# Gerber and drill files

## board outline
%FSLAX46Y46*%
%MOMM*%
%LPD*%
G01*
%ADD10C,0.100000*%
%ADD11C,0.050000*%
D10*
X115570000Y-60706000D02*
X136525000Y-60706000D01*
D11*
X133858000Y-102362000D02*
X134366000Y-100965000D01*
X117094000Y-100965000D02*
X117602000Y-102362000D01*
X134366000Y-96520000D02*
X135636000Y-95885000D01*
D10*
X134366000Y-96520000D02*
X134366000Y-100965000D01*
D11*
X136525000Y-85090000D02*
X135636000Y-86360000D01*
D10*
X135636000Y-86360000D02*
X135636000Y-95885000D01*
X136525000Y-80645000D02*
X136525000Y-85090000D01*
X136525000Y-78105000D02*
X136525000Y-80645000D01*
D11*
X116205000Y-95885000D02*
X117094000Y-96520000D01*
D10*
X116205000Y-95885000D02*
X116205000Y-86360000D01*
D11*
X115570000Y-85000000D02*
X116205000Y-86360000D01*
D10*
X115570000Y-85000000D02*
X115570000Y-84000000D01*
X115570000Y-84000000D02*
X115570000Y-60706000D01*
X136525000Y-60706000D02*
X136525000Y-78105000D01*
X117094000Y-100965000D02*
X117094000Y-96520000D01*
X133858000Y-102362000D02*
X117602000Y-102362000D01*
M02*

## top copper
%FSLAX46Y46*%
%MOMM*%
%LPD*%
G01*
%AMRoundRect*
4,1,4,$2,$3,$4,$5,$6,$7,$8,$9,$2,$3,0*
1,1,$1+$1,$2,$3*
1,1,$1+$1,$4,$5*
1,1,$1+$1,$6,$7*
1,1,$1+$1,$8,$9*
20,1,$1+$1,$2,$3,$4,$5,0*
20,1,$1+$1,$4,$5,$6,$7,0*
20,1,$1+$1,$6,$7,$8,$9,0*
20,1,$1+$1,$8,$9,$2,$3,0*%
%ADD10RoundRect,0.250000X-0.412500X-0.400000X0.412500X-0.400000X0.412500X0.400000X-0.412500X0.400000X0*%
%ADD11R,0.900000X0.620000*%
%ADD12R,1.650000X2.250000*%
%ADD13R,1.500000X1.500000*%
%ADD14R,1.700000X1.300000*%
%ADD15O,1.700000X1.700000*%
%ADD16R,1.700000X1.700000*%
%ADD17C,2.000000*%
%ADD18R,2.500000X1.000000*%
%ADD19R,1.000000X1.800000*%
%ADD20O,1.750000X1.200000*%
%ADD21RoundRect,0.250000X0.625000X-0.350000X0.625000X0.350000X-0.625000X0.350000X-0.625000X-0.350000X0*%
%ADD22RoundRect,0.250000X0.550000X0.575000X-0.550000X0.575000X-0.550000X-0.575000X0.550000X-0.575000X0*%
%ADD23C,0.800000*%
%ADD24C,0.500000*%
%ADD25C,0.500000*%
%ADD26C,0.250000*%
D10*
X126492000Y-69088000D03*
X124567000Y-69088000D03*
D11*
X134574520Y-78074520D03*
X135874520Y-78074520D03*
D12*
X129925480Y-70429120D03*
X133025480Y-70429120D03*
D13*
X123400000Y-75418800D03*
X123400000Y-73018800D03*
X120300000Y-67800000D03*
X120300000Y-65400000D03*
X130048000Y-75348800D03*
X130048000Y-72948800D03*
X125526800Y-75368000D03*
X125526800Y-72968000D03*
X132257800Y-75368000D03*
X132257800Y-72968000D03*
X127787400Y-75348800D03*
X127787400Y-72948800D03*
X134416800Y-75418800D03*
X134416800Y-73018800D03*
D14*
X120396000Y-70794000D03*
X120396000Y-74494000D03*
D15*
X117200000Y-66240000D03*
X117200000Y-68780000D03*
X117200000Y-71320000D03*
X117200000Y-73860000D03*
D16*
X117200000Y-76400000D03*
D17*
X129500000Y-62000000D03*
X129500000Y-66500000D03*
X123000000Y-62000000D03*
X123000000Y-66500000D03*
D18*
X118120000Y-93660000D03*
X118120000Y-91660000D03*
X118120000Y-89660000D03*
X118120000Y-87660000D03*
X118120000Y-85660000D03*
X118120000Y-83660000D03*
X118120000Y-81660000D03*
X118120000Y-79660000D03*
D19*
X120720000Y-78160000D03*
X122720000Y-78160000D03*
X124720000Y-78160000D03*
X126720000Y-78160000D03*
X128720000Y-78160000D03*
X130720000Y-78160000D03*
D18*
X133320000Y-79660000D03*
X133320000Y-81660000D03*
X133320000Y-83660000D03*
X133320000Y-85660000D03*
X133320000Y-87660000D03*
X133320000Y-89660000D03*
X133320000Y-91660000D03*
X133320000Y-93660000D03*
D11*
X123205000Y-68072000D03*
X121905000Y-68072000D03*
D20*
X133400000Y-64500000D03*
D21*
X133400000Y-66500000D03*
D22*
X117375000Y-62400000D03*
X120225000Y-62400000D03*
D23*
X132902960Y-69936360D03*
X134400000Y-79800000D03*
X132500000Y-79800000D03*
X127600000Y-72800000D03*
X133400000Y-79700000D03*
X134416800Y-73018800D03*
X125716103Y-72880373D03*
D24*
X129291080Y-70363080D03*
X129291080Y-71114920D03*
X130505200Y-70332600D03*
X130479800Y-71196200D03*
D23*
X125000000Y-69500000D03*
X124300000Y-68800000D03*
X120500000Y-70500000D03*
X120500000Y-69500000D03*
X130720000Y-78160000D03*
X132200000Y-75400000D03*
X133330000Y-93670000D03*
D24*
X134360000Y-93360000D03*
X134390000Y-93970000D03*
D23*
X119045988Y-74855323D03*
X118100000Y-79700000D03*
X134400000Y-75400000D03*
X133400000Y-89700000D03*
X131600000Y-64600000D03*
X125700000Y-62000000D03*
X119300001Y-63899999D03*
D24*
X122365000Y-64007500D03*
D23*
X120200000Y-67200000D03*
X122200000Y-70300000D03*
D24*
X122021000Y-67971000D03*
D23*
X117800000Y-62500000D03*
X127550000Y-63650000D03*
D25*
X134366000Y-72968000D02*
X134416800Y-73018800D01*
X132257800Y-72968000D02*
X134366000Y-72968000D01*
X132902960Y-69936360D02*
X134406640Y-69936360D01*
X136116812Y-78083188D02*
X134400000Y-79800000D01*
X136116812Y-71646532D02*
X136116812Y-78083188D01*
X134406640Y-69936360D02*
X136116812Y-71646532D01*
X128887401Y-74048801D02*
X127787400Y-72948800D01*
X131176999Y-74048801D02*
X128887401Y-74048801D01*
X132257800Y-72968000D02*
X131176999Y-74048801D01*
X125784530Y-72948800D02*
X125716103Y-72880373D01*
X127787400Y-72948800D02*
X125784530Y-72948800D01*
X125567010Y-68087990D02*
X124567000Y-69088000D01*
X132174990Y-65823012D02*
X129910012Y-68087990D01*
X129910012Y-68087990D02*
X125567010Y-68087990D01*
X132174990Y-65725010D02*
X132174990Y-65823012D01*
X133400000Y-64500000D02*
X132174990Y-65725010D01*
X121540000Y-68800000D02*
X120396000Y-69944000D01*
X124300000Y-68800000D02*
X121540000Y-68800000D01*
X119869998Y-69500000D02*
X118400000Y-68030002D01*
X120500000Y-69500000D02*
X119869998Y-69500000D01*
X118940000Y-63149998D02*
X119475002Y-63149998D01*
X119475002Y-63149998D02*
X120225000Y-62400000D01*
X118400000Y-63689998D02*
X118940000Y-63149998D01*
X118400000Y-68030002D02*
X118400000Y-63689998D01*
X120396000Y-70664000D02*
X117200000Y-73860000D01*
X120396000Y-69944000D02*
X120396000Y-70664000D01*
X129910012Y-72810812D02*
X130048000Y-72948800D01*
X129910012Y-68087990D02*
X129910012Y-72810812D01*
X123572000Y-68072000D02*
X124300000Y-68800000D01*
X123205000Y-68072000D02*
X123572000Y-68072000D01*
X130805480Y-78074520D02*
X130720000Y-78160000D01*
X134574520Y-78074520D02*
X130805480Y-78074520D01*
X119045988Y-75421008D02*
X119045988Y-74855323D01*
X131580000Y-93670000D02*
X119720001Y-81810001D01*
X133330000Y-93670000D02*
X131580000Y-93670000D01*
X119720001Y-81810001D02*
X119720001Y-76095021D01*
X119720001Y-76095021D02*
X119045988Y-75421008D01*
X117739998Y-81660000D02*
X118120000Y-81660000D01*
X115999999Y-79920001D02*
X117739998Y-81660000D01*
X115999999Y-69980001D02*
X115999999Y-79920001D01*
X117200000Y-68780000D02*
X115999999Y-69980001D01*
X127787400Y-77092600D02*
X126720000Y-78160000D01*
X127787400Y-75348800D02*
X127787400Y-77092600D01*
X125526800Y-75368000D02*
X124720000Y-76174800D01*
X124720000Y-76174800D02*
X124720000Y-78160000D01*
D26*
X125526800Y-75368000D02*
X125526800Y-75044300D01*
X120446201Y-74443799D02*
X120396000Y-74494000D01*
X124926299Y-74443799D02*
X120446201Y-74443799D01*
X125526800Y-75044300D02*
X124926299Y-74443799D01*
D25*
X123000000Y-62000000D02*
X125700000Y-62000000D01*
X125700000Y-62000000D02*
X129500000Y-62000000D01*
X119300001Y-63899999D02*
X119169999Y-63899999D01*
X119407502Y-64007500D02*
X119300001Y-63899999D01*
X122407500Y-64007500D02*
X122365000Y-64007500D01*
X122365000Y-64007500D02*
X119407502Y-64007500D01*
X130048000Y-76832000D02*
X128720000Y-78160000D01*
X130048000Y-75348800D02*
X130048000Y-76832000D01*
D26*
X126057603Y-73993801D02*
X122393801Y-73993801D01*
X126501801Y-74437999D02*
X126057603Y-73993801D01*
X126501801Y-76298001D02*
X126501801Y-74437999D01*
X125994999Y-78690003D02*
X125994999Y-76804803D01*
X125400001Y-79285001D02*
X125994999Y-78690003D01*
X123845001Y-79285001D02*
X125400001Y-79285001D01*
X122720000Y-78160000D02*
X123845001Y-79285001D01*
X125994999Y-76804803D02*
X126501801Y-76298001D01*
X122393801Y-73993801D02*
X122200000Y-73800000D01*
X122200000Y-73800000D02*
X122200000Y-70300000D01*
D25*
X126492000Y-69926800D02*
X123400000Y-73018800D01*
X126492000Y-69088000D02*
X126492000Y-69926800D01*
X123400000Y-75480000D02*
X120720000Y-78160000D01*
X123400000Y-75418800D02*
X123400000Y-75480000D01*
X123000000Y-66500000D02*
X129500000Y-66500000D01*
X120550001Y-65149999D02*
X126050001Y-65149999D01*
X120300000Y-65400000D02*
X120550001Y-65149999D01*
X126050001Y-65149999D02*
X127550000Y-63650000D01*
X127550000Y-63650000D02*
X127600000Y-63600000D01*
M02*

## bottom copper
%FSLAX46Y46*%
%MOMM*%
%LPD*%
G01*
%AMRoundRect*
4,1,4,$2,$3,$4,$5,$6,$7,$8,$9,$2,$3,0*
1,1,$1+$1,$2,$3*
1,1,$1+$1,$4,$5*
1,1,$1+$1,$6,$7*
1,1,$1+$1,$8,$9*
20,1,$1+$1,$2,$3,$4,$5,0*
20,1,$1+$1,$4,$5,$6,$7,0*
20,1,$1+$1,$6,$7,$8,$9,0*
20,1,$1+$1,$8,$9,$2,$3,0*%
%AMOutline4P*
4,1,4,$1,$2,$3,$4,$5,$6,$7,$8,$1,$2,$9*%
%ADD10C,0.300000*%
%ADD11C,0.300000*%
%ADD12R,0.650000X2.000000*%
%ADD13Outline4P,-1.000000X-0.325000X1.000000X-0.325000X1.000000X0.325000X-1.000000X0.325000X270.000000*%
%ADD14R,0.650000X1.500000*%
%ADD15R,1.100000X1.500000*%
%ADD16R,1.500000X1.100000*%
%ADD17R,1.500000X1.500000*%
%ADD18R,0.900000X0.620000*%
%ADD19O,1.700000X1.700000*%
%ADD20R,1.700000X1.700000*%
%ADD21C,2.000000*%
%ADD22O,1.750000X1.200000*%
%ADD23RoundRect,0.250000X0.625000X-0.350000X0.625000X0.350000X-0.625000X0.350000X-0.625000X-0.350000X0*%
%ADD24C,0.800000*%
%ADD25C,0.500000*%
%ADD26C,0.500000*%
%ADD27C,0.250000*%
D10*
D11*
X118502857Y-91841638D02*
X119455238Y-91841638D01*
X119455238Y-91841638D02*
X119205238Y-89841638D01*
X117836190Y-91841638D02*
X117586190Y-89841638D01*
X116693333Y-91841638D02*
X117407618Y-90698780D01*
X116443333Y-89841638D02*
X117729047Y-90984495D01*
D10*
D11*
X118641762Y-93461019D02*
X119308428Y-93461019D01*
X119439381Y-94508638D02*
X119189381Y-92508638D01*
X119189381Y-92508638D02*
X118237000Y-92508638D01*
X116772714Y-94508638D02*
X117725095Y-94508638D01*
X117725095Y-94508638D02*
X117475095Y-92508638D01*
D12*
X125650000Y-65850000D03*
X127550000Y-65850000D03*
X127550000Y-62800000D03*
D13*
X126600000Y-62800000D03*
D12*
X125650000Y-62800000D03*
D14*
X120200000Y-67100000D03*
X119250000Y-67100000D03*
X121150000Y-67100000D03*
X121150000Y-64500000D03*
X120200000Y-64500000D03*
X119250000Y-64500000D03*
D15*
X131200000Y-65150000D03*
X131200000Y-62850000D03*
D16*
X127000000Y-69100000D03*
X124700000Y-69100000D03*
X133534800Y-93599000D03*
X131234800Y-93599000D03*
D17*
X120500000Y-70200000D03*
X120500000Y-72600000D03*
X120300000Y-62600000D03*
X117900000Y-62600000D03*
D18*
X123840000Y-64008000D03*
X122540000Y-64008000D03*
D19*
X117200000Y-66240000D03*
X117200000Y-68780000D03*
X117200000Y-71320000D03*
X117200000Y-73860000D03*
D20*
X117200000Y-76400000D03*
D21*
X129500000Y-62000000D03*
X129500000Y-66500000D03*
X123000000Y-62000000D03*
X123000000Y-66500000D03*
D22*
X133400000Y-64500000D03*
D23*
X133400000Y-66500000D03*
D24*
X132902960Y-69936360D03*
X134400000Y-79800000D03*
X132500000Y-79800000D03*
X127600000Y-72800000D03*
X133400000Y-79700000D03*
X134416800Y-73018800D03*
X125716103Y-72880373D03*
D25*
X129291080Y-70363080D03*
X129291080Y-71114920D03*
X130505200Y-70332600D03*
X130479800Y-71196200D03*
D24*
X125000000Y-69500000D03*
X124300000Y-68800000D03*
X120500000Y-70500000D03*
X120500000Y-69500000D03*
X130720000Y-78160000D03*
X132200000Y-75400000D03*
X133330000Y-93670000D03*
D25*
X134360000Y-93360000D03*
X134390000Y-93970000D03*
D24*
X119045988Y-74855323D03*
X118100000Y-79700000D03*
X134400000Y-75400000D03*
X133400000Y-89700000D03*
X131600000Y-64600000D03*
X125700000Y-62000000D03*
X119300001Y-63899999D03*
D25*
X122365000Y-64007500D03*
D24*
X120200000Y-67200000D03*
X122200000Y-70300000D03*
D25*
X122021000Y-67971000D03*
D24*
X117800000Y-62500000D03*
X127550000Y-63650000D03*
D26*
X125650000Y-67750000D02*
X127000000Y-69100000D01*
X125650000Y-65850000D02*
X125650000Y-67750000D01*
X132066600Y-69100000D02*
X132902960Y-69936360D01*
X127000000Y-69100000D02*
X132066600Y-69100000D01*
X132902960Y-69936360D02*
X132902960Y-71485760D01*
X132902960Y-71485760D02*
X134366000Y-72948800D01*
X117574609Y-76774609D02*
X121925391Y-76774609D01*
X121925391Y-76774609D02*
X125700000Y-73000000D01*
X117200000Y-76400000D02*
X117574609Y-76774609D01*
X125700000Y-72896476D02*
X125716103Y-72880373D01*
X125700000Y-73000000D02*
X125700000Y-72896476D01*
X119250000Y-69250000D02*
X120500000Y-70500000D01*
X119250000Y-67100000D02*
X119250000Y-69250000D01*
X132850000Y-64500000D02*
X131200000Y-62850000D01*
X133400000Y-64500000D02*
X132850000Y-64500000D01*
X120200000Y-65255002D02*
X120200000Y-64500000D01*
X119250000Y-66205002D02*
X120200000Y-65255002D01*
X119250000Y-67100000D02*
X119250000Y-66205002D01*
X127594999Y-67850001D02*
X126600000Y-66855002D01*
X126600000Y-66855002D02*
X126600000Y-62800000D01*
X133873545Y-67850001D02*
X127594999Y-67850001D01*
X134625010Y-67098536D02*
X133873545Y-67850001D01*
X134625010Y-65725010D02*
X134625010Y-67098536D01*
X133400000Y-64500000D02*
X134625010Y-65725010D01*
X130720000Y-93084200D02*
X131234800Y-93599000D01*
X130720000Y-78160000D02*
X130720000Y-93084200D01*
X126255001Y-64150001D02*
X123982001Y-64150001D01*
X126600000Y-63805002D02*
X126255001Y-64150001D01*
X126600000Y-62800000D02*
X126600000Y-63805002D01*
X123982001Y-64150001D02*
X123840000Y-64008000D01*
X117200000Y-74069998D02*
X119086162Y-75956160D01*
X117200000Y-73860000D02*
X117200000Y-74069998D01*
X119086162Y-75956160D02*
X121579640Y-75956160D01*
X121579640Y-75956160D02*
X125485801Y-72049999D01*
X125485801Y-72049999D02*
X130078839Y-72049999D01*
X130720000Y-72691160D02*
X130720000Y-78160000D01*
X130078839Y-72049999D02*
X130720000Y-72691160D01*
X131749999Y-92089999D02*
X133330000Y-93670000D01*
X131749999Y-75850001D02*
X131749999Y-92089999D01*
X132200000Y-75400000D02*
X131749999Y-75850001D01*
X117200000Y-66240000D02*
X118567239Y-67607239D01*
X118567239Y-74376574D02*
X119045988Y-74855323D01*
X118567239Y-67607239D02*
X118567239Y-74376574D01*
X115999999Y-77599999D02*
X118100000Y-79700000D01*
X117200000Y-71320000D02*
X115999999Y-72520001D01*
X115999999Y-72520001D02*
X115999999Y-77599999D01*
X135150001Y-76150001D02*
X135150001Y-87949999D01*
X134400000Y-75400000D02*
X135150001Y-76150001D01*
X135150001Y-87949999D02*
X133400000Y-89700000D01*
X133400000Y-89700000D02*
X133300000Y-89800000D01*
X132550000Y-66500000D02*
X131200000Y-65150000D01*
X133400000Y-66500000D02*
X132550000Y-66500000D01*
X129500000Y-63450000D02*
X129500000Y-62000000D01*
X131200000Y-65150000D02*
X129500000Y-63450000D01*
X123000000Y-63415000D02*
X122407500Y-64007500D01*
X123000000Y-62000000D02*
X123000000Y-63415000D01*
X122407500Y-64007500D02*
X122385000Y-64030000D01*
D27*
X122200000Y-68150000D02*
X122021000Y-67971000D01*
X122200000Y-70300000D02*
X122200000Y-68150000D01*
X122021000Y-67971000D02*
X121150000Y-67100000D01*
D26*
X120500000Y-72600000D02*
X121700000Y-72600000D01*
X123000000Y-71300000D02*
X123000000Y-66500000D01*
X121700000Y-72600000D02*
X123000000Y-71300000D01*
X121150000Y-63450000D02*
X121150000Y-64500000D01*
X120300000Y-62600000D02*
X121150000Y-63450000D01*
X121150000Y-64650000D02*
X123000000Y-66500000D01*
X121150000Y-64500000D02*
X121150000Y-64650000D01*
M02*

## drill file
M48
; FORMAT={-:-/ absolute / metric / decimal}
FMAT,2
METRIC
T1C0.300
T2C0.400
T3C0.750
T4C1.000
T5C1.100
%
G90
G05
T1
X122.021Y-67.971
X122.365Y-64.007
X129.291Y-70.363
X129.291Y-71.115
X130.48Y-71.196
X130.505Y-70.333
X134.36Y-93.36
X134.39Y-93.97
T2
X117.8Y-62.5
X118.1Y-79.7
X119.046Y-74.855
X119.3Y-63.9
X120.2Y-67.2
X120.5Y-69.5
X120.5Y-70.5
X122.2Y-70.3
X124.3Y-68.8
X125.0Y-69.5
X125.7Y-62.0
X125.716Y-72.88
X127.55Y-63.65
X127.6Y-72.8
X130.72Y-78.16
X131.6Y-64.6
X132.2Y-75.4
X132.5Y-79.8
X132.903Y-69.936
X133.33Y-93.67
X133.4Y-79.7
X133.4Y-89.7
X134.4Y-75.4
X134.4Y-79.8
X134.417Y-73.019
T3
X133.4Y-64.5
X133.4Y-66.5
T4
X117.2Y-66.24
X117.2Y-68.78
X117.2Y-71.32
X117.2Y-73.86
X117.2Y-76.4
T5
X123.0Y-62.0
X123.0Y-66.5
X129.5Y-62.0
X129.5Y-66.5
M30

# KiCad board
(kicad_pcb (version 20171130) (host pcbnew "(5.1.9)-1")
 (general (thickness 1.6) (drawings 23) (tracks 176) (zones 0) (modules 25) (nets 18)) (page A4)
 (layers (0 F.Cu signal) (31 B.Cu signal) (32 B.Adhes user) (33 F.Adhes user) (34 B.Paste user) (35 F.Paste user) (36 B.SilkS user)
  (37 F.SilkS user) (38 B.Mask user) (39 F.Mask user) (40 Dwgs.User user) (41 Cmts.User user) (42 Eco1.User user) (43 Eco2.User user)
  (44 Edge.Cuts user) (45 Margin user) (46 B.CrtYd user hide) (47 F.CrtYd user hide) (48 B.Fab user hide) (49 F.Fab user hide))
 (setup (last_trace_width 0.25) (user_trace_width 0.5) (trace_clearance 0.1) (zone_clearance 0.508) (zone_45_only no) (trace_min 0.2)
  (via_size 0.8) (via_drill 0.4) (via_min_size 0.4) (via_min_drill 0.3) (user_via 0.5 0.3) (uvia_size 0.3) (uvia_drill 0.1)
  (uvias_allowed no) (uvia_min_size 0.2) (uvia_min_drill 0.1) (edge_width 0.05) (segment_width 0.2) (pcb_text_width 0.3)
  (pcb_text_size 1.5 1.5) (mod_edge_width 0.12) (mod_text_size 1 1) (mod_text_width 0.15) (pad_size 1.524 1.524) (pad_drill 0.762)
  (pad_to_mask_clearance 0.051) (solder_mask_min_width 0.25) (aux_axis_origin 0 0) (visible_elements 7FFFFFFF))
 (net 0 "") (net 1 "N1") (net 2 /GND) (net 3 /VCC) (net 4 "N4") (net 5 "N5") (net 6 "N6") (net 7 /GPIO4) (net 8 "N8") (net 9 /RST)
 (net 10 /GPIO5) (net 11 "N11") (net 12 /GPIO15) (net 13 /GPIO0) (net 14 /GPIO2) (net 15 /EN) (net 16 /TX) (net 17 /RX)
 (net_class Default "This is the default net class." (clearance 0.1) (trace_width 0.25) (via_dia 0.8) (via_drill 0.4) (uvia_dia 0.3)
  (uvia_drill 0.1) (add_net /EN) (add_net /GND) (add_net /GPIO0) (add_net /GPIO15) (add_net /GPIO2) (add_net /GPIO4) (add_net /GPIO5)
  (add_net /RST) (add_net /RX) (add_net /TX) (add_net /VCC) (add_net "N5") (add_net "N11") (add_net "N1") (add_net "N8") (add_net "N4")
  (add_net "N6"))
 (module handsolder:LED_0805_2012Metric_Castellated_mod (layer F.Cu) (at 125.5295 69.088)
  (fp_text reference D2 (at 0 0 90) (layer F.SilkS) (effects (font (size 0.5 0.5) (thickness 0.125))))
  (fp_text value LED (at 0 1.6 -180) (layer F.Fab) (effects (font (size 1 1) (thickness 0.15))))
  (pad 2 smd roundrect (at 0.9625 0) (size 1.325 1.3) (layers F.Cu F.Paste F.Mask) (roundrect_rratio 0.1923076923076923) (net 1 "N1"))
  (pad 1 smd roundrect (at -0.9625 0) (size 1.325 1.3) (layers F.Cu F.Paste F.Mask) (roundrect_rratio 0.1923076923076923) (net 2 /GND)))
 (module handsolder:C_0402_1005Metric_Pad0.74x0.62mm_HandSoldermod (layer F.Cu) (at 135.22452 78.07452 180)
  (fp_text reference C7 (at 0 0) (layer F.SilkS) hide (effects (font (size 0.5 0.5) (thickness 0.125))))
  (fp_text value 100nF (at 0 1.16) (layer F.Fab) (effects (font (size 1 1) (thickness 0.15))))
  (pad 2 smd rect (at 0.65 0 180) (size 0.9 0.62) (layers F.Cu F.Paste F.Mask) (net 2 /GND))
  (pad 1 smd rect (at -0.65 0 180) (size 0.9 0.62) (layers F.Cu F.Paste F.Mask) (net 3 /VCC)))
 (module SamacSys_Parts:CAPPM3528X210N (layer F.Cu) (at 131.47548 70.42912 180)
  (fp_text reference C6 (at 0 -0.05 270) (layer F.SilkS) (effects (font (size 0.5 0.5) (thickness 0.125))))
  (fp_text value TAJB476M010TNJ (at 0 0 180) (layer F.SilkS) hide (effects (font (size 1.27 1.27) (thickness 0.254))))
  (pad 2 smd rect (at 1.55 0 180) (size 1.65 2.25) (layers F.Cu F.Paste F.Mask) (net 2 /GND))
  (pad 1 smd rect (at -1.55 0 180) (size 1.65 2.25) (layers F.Cu F.Paste F.Mask) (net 3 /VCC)))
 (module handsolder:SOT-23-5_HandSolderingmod (layer B.Cu) (at 126.6 64.35 270)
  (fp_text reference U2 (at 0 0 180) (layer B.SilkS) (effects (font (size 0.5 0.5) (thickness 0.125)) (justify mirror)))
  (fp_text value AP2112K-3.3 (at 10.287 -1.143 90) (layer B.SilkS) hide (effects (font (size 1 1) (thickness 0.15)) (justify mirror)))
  (pad 5 smd rect (at 1.5 0.95 270) (size 2 0.65) (layers B.Cu B.Paste B.Mask) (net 3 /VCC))
  (pad 4 smd rect (at 1.5 -0.95 270) (size 2 0.65) (layers B.Cu B.Paste B.Mask))
  (pad 3 smd rect (at -1.55 -0.95 270) (size 2 0.65) (layers B.Cu B.Paste B.Mask) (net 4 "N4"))
  (pad 2 smd trapezoid (at -1.55 0 270) (size 2 0.65) (layers B.Cu B.Paste B.Mask) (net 2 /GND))
  (pad 1 smd rect (at -1.55 0.95 270) (size 2 0.65) (layers B.Cu B.Paste B.Mask) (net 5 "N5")))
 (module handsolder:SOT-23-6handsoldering (layer B.Cu) (at 120.2 65.8 270)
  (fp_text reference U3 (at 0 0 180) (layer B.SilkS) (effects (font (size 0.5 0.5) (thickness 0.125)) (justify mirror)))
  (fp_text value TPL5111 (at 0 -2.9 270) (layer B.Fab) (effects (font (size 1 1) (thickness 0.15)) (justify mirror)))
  (pad 5 smd rect (at 1.3 0 270) (size 1.5 0.65) (layers B.Cu B.Paste B.Mask) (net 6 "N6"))
  (pad 6 smd rect (at 1.3 0.95 270) (size 1.5 0.65) (layers B.Cu B.Paste B.Mask) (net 2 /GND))
  (pad 4 smd rect (at 1.3 -0.95 270) (size 1.5 0.65) (layers B.Cu B.Paste B.Mask) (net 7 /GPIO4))
  (pad 3 smd rect (at -1.3 -0.95 270) (size 1.5 0.65) (layers B.Cu B.Paste B.Mask) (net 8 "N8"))
  (pad 2 smd rect (at -1.3 0 270) (size 1.5 0.65) (layers B.Cu B.Paste B.Mask) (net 2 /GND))
  (pad 1 smd rect (at -1.3 0.95 270) (size 1.5 0.65) (layers B.Cu B.Paste B.Mask) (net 5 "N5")))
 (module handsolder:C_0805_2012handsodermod (layer B.Cu) (at 131.2 64 270)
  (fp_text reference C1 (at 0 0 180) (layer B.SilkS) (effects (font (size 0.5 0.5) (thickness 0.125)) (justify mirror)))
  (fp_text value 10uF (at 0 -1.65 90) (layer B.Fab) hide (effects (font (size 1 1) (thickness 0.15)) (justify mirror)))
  (pad 2 smd rect (at 1.15 0 270) (size 1.5 1.1) (layers B.Cu B.Paste B.Mask) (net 5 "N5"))
  (pad 1 smd rect (at -1.15 0 270) (size 1.5 1.1) (layers B.Cu B.Paste B.Mask) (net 2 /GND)))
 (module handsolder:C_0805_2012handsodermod (layer B.Cu) (at 125.85 69.1)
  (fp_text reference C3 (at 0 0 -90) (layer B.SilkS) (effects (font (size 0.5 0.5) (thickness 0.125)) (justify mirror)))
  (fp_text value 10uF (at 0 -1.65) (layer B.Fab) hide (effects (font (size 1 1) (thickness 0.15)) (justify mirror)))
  (pad 2 smd rect (at 1.15 0) (size 1.5 1.1) (layers B.Cu B.Paste B.Mask) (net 3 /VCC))
  (pad 1 smd rect (at -1.15 0) (size 1.5 1.1) (layers B.Cu B.Paste B.Mask) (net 2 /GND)))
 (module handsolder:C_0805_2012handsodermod (layer B.Cu) (at 132.3848 93.599)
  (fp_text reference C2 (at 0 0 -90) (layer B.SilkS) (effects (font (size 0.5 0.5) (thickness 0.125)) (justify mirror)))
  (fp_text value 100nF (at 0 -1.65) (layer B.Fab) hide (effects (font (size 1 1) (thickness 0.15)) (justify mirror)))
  (pad 2 smd rect (at 1.15 0) (size 1.5 1.1) (layers B.Cu B.Paste B.Mask) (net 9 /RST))
  (pad 1 smd rect (at -1.15 0) (size 1.5 1.1) (layers B.Cu B.Paste B.Mask) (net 2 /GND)))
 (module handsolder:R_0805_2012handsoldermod (layer B.Cu) (at 120.5 71.4 90)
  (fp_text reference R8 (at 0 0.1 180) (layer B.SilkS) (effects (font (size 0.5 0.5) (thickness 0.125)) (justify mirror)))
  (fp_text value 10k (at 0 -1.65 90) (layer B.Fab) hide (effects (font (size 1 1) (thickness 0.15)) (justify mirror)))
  (pad 2 smd rect (at 1.2 0 90) (size 1.5 1.5) (layers B.Cu B.Paste B.Mask) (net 2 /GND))
  (pad 1 smd rect (at -1.2 0 90) (size 1.5 1.5) (layers B.Cu B.Paste B.Mask) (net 8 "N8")))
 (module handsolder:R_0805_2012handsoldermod (layer F.Cu) (at 123.4 74.2188 270)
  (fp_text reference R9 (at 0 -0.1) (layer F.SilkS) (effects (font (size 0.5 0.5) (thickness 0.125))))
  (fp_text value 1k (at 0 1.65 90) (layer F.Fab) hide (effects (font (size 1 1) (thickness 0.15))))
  (pad 2 smd rect (at 1.2 0 270) (size 1.5 1.5) (layers F.Cu F.Paste F.Mask) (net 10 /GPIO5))
  (pad 1 smd rect (at -1.2 0 270) (size 1.5 1.5) (layers F.Cu F.Paste F.Mask) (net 1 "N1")))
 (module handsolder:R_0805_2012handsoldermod (layer F.Cu) (at 120.3 66.6 270)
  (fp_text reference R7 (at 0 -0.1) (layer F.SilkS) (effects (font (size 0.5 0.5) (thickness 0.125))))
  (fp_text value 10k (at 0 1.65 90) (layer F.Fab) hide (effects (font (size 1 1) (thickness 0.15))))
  (pad 2 smd rect (at 1.2 0 270) (size 1.5 1.5) (layers F.Cu F.Paste F.Mask) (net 6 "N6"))
  (pad 1 smd rect (at -1.2 0 270) (size 1.5 1.5) (layers F.Cu F.Paste F.Mask) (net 4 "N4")))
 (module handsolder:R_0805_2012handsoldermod (layer B.Cu) (at 119.1 62.6)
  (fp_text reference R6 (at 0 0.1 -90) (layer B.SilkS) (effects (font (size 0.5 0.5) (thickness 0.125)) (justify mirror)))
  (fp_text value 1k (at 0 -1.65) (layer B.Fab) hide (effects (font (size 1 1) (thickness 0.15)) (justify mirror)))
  (pad 2 smd rect (at 1.2 0) (size 1.5 1.5) (layers B.Cu B.Paste B.Mask) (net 8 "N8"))
  (pad 1 smd rect (at -1.2 0) (size 1.5 1.5) (layers B.Cu B.Paste B.Mask) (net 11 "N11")))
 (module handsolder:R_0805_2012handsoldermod (layer F.Cu) (at 130.048 74.1488 270)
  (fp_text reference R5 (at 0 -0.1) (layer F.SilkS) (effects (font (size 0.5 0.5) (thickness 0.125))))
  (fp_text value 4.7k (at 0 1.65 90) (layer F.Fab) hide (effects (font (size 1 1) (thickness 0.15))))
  (pad 2 smd rect (at 1.2 0 270) (size 1.5 1.5) (layers F.Cu F.Paste F.Mask) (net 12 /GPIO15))
  (pad 1 smd rect (at -1.2 0 270) (size 1.5 1.5) (layers F.Cu F.Paste F.Mask) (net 2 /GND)))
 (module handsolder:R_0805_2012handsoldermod (layer F.Cu) (at 125.5268 74.168 270)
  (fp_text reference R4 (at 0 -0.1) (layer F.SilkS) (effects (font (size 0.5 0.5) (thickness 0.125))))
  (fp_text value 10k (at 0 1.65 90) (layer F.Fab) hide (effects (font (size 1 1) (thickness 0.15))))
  (pad 2 smd rect (at 1.2 0 270) (size 1.5 1.5) (layers F.Cu F.Paste F.Mask) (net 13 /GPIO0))
  (pad 1 smd rect (at -1.2 0 270) (size 1.5 1.5) (layers F.Cu F.Paste F.Mask) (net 3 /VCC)))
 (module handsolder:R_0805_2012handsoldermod (layer F.Cu) (at 132.2578 74.168 270)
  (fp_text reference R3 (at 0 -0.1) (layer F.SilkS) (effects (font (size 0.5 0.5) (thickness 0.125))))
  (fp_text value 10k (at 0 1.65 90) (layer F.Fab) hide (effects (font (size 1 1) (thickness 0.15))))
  (pad 2 smd rect (at 1.2 0 270) (size 1.5 1.5) (layers F.Cu F.Paste F.Mask) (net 9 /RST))
  (pad 1 smd rect (at -1.2 0 270) (size 1.5 1.5) (layers F.Cu F.Paste F.Mask) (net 3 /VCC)))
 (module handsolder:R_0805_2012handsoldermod (layer F.Cu) (at 127.7874 74.1488 270)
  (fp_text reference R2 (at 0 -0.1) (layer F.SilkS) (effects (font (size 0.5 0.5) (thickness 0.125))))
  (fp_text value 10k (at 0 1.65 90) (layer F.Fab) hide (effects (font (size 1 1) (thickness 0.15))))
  (pad 2 smd rect (at 1.2 0 270) (size 1.5 1.5) (layers F.Cu F.Paste F.Mask) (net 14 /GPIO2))
  (pad 1 smd rect (at -1.2 0 270) (size 1.5 1.5) (layers F.Cu F.Paste F.Mask) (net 3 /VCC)))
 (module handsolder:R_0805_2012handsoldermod (layer F.Cu) (at 134.4168 74.2188 270)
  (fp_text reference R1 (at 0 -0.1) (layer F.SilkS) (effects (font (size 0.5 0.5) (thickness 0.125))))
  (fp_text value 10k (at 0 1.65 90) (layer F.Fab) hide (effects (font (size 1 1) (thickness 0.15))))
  (pad 2 smd rect (at 1.2 0 270) (size 1.5 1.5) (layers F.Cu F.Paste F.Mask) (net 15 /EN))
  (pad 1 smd rect (at -1.2 0 270) (size 1.5 1.5) (layers F.Cu F.Paste F.Mask) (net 3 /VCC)))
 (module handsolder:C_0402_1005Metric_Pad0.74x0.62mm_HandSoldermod (layer B.Cu) (at 123.19 64.008)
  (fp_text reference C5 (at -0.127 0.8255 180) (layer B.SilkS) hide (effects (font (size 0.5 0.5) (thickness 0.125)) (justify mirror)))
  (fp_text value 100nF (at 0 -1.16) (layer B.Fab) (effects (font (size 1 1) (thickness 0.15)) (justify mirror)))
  (pad 2 smd rect (at 0.65 0) (size 0.9 0.62) (layers B.Cu B.Paste B.Mask) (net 2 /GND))
  (pad 1 smd rect (at -0.65 0) (size 0.9 0.62) (layers B.Cu B.Paste B.Mask) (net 5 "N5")))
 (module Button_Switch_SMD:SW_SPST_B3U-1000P (layer F.Cu) (at 120.396 72.644 90)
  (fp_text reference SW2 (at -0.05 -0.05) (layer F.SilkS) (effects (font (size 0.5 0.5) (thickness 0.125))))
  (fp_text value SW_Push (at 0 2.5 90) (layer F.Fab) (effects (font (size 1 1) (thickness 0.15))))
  (pad 2 smd rect (at 1.85 0 90) (size 1.3 1.7) (layers F.Cu F.Paste F.Mask) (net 2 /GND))
  (pad 1 smd rect (at -1.85 0 90) (size 1.3 1.7) (layers F.Cu F.Paste F.Mask) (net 13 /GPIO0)))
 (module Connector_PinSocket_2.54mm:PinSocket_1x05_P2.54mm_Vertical (layer F.Cu) (at 117.2 76.4 180)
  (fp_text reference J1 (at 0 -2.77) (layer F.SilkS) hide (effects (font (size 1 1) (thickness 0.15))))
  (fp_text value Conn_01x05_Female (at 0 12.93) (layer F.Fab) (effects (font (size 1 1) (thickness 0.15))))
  (pad 5 thru_hole oval (at 0 10.16 180) (size 1.7 1.7) (drill 1) (layers *.Cu *.Mask) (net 9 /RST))
  (pad 4 thru_hole oval (at 0 7.62 180) (size 1.7 1.7) (drill 1) (layers *.Cu *.Mask) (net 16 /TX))
  (pad 3 thru_hole oval (at 0 5.08 180) (size 1.7 1.7) (drill 1) (layers *.Cu *.Mask) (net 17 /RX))
  (pad 2 thru_hole oval (at 0 2.54 180) (size 1.7 1.7) (drill 1) (layers *.Cu *.Mask) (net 2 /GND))
  (pad 1 thru_hole rect (at 0 0 180) (size 1.7 1.7) (drill 1) (layers *.Cu *.Mask) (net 3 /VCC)))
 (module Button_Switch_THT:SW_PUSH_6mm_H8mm (layer F.Cu) (at 123 62)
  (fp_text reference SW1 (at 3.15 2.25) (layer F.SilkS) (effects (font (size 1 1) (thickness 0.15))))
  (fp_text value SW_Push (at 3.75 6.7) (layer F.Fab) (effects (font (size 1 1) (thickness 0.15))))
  (pad 1 thru_hole circle (at 6.5 0 90) (size 2 2) (drill 1.1) (layers *.Cu *.Mask) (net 5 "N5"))
  (pad 2 thru_hole circle (at 6.5 4.5 90) (size 2 2) (drill 1.1) (layers *.Cu *.Mask) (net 8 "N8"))
  (pad 1 thru_hole circle (at 0 0 90) (size 2 2) (drill 1.1) (layers *.Cu *.Mask) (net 5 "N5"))
  (pad 2 thru_hole circle (at 0 4.5 90) (size 2 2) (drill 1.1) (layers *.Cu *.Mask) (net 8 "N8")))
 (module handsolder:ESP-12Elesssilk (layer F.Cu) (at 125.72 90.16 180)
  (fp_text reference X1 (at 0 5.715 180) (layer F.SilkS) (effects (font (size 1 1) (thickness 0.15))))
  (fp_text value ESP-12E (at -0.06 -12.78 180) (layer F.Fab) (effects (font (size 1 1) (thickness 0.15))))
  (pad 22 smd rect (at 7.6 -3.5 180) (size 2.5 1) (layers F.Cu F.Paste F.Mask))
  (pad 21 smd rect (at 7.6 -1.5 180) (size 2.5 1) (layers F.Cu F.Paste F.Mask))
  (pad 20 smd rect (at 7.6 0.5 180) (size 2.5 1) (layers F.Cu F.Paste F.Mask))
  (pad 19 smd rect (at 7.6 2.5 180) (size 2.5 1) (layers F.Cu F.Paste F.Mask))
  (pad 18 smd rect (at 7.6 4.5 180) (size 2.5 1) (layers F.Cu F.Paste F.Mask))
  (pad 17 smd rect (at 7.6 6.5 180) (size 2.5 1) (layers F.Cu F.Paste F.Mask))
  (pad 16 smd rect (at 7.6 8.5 180) (size 2.5 1) (layers F.Cu F.Paste F.Mask) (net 16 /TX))
  (pad 15 smd rect (at 7.6 10.5 180) (size 2.5 1) (layers F.Cu F.Paste F.Mask) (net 17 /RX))
  (pad 14 smd rect (at 5 12 180) (size 1 1.8) (layers F.Cu F.Paste F.Mask) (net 10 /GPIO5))
  (pad 13 smd rect (at 3 12 180) (size 1 1.8) (layers F.Cu F.Paste F.Mask) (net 7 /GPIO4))
  (pad 12 smd rect (at 1 12 180) (size 1 1.8) (layers F.Cu F.Paste F.Mask) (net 13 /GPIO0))
  (pad 11 smd rect (at -1 12 180) (size 1 1.8) (layers F.Cu F.Paste F.Mask) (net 14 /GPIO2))
  (pad 10 smd rect (at -3 12 180) (size 1 1.8) (layers F.Cu F.Paste F.Mask) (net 12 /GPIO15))
  (pad 9 smd rect (at -5 12 180) (size 1 1.8) (layers F.Cu F.Paste F.Mask) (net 2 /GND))
  (pad 8 smd rect (at -7.6 10.5 180) (size 2.5 1) (layers F.Cu F.Paste F.Mask) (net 3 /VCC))
  (pad 7 smd rect (at -7.6 8.5 180) (size 2.5 1) (layers F.Cu F.Paste F.Mask))
  (pad 6 smd rect (at -7.6 6.5 180) (size 2.5 1) (layers F.Cu F.Paste F.Mask))
  (pad 5 smd rect (at -7.6 4.5 180) (size 2.5 1) (layers F.Cu F.Paste F.Mask))
  (pad 4 smd rect (at -7.6 2.5 180) (size 2.5 1) (layers F.Cu F.Paste F.Mask))
  (pad 3 smd rect (at -7.6 0.5 180) (size 2.5 1) (layers F.Cu F.Paste F.Mask) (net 15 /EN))
  (pad 2 smd rect (at -7.6 -1.5 180) (size 2.5 1) (layers F.Cu F.Paste F.Mask))
  (pad 1 smd rect (at -7.6 -3.5 180) (size 2.5 1) (layers F.Cu F.Paste F.Mask) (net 9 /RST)))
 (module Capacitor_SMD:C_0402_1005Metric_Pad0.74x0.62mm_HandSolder (layer F.Cu) (at 122.555 68.072)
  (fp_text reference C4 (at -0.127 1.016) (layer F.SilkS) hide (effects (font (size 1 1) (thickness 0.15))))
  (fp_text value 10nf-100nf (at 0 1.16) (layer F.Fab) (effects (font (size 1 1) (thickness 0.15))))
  (pad 2 smd rect (at 0.65 0) (size 0.9 0.62) (layers F.Cu F.Paste F.Mask) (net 2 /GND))
  (pad 1 smd rect (at -0.65 0) (size 0.9 0.62) (layers F.Cu F.Paste F.Mask) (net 7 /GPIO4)))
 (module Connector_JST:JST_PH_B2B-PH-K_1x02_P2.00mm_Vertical (layer F.Cu) (at 133.4 66.5 90)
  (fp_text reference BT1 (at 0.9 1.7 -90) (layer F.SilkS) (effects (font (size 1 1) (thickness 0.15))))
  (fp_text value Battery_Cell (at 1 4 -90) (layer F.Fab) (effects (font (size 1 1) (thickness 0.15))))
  (pad 2 thru_hole oval (at 2 0 90) (size 1.2 1.75) (drill 0.75) (layers *.Cu *.Mask) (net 2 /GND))
  (pad 1 thru_hole roundrect (at 0 0 90) (size 1.2 1.75) (drill 0.75) (layers *.Cu *.Mask) (roundrect_rratio 0.208333) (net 5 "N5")))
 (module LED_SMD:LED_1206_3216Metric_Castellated (layer F.Cu) (at 118.8 62.4 180)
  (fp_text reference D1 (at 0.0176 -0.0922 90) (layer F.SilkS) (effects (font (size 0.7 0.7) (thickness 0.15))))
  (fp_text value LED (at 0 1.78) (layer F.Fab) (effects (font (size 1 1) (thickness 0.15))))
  (pad 2 smd roundrect (at 1.425 0 180) (size 1.6 1.65) (layers F.Cu F.Paste F.Mask) (roundrect_rratio 0.15625) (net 11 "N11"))
  (pad 1 smd roundrect (at -1.425 0 180) (size 1.6 1.65) (layers F.Cu F.Paste F.Mask) (roundrect_rratio 0.15625) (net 2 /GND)))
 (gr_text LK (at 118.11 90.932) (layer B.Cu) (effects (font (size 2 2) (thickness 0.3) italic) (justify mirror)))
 (gr_line (start 115.57 60.706) (end 136.525 60.706) (layer Edge.Cuts) (width 0.1))
 (gr_line (start 133.858 102.362) (end 134.366 100.965) (layer Edge.Cuts) (width 0.05))
 (gr_line (start 117.094 100.965) (end 117.602 102.362) (layer Edge.Cuts) (width 0.05))
 (gr_line (start 134.366 96.52) (end 135.636 95.885) (layer Edge.Cuts) (width 0.05))
 (gr_line (start 134.366 96.52) (end 134.366 100.965) (layer Edge.Cuts) (width 0.1))
 (gr_line (start 136.525 85.09) (end 135.636 86.36) (layer Edge.Cuts) (width 0.05))
 (gr_line (start 135.636 86.36) (end 135.636 95.885) (layer Edge.Cuts) (width 0.1))
 (gr_line (start 136.525 80.645) (end 136.525 85.09) (layer Edge.Cuts) (width 0.1))
 (gr_line (start 136.525 78.105) (end 136.525 80.645) (layer Edge.Cuts) (width 0.1))
 (gr_line (start 116.205 95.885) (end 117.094 96.52) (layer Edge.Cuts) (width 0.05))
 (gr_line (start 116.205 95.885) (end 116.205 86.36) (layer Edge.Cuts) (width 0.1))
 (gr_line (start 115.57 85) (end 116.205 86.36) (layer Edge.Cuts) (width 0.05))
 (gr_line (start 115.57 85) (end 115.57 84) (layer Edge.Cuts) (width 0.1))
 (gr_line (start 115.57 84) (end 115.57 60.706) (layer Edge.Cuts) (width 0.1))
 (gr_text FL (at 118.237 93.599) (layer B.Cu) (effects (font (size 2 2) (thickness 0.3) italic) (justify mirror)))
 (gr_line (start 136.525 60.706) (end 136.525 78.105) (layer Edge.Cuts) (width 0.1))
 (gr_line (start 117.094 100.965) (end 117.094 96.52) (layer Edge.Cuts) (width 0.1))
 (gr_line (start 133.858 102.362) (end 117.602 102.362) (layer Edge.Cuts) (width 0.1))
 (via (at 132.90296 69.93636) (size 0.8) (drill 0.4) (layers F.Cu B.Cu) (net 3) (status 30))
 (via (at 134.4 79.8) (size 0.8) (drill 0.4) (layers F.Cu B.Cu) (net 3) (status 30))
 (via (at 132.5 79.8) (size 0.8) (drill 0.4) (layers F.Cu B.Cu) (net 3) (status 30))
 (segment (start 125.65 67.75) (end 127 69.1) (width 0.5) (layer B.Cu) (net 3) (status 20))
 (segment (start 125.65 65.85) (end 125.65 67.75) (width 0.5) (layer B.Cu) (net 3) (status 10))
 (segment (start 134.366 72.968) (end 134.4168 73.0188) (width 0.5) (layer F.Cu) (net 3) (status 30))
 (segment (start 132.2578 72.968) (end 134.366 72.968) (width 0.5) (layer F.Cu) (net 3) (status 30))
 (via (at 127.6 72.8) (size 0.8) (drill 0.4) (layers F.Cu B.Cu) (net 3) (status 30))
 (via (at 133.4 79.7) (size 0.8) (drill 0.4) (layers F.Cu B.Cu) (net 3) (status 30))
 (segment (start 132.0666 69.1) (end 132.90296 69.93636) (width 0.5) (layer B.Cu) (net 3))
 (segment (start 127 69.1) (end 132.0666 69.1) (width 0.5) (layer B.Cu) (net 3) (status 10))
 (segment (start 132.90296 69.93636) (end 132.90296 71.48576) (width 0.5) (layer B.Cu) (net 3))
 (segment (start 132.90296 71.48576) (end 134.366 72.9488) (width 0.5) (layer B.Cu) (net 3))
 (via (at 134.4168 73.0188) (size 0.8) (drill 0.4) (layers F.Cu B.Cu) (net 3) (status 30))
 (segment (start 132.90296 69.93636) (end 134.40664 69.93636) (width 0.5) (layer F.Cu) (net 3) (status 10))
 (segment (start 136.116812 78.083188) (end 134.4 79.8) (width 0.5) (layer F.Cu) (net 3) (status 20))
 (segment (start 136.116812 71.646532) (end 136.116812 78.083188) (width 0.5) (layer F.Cu) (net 3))
 (segment (start 134.40664 69.93636) (end 136.116812 71.646532) (width 0.5) (layer F.Cu) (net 3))
 (segment (start 128.887401 74.048801) (end 127.7874 72.9488) (width 0.5) (layer F.Cu) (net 3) (status 20))
 (segment (start 131.176999 74.048801) (end 128.887401 74.048801) (width 0.5) (layer F.Cu) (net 3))
 (segment (start 132.2578 72.968) (end 131.176999 74.048801) (width 0.5) (layer F.Cu) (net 3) (status 10))
 (via (at 125.716103 72.880373) (size 0.8) (drill 0.4) (layers F.Cu B.Cu) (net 3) (status 30))
 (segment (start 117.574609 76.774609) (end 121.925391 76.774609) (width 0.5) (layer B.Cu) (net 3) (status 10))
 (segment (start 121.925391 76.774609) (end 125.7 73) (width 0.5) (layer B.Cu) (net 3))
 (segment (start 117.2 76.4) (end 117.574609 76.774609) (width 0.5) (layer B.Cu) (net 3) (status 30))
 (segment (start 125.7 72.896476) (end 125.716103 72.880373) (width 0.5) (layer B.Cu) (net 3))
 (segment (start 125.7 73) (end 125.7 72.896476) (width 0.5) (layer B.Cu) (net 3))
 (segment (start 125.78453 72.9488) (end 125.716103 72.880373) (width 0.5) (layer F.Cu) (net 3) (status 30))
 (segment (start 127.7874 72.9488) (end 125.78453 72.9488) (width 0.5) (layer F.Cu) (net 3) (status 30))
 (via (at 129.29108 70.36308) (size 0.5) (drill 0.3) (layers F.Cu B.Cu) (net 2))
 (via (at 129.29108 71.11492) (size 0.5) (drill 0.3) (layers F.Cu B.Cu) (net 2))
 (via (at 130.5052 70.3326) (size 0.5) (drill 0.3) (layers F.Cu B.Cu) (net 2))
 (via (at 130.4798 71.1962) (size 0.5) (drill 0.3) (layers F.Cu B.Cu) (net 2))
 (via (at 125 69.5) (size 0.8) (drill 0.4) (layers F.Cu B.Cu) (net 2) (status 30))
 (via (at 124.3 68.8) (size 0.8) (drill 0.4) (layers F.Cu B.Cu) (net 2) (status 30))
 (via (at 120.5 70.5) (size 0.8) (drill 0.4) (layers F.Cu B.Cu) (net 2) (status 30))
 (via (at 120.5 69.5) (size 0.8) (drill 0.4) (layers F.Cu B.Cu) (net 2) (status 30))
 (segment (start 119.25 69.25) (end 120.5 70.5) (width 0.5) (layer B.Cu) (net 2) (status 20))
 (segment (start 119.25 67.1) (end 119.25 69.25) (width 0.5) (layer B.Cu) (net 2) (status 10))
 (segment (start 132.85 64.5) (end 131.2 62.85) (width 0.5) (layer B.Cu) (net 2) (status 30))
 (segment (start 133.4 64.5) (end 132.85 64.5) (width 0.5) (layer B.Cu) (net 2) (status 30))
 (segment (start 120.2 65.255002) (end 120.2 64.5) (width 0.5) (layer B.Cu) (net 2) (status 20))
 (segment (start 119.25 66.205002) (end 120.2 65.255002) (width 0.5) (layer B.Cu) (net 2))
 (segment (start 119.25 67.1) (end 119.25 66.205002) (width 0.5) (layer B.Cu) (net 2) (status 10))
 (segment (start 127.594999 67.850001) (end 126.6 66.855002) (width 0.5) (layer B.Cu) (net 2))
 (segment (start 126.6 66.855002) (end 126.6 62.8) (width 0.5) (layer B.Cu) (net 2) (status 20))
 (segment (start 133.873545 67.850001) (end 127.594999 67.850001) (width 0.5) (layer B.Cu) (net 2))
 (segment (start 134.62501 67.098536) (end 133.873545 67.850001) (width 0.5) (layer B.Cu) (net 2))
 (segment (start 134.62501 65.72501) (end 134.62501 67.098536) (width 0.5) (layer B.Cu) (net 2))
 (segment (start 133.4 64.5) (end 134.62501 65.72501) (width 0.5) (layer B.Cu) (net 2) (status 10))
 (segment (start 125.56701 68.08799) (end 124.567 69.088) (width 0.5) (layer F.Cu) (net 2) (status 20))
 (segment (start 132.17499 65.823012) (end 129.910012 68.08799) (width 0.5) (layer F.Cu) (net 2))
 (segment (start 129.910012 68.08799) (end 125.56701 68.08799) (width 0.5) (layer F.Cu) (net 2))
 (segment (start 132.17499 65.72501) (end 132.17499 65.823012) (width 0.5) (layer F.Cu) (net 2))
 (segment (start 133.4 64.5) (end 132.17499 65.72501) (width 0.5) (layer F.Cu) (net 2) (status 10))
 (segment (start 121.54 68.8) (end 120.396 69.944) (width 0.5) (layer F.Cu) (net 2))
 (segment (start 124.3 68.8) (end 121.54 68.8) (width 0.5) (layer F.Cu) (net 2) (status 10))
 (segment (start 119.869998 69.5) (end 118.4 68.030002) (width 0.5) (layer F.Cu) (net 2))
 (segment (start 120.5 69.5) (end 119.869998 69.5) (width 0.5) (layer F.Cu) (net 2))
 (segment (start 118.94 63.149998) (end 119.475002 63.149998) (width 0.5) (layer F.Cu) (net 2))
 (segment (start 119.475002 63.149998) (end 120.225 62.4) (width 0.5) (layer F.Cu) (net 2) (status 20))
 (segment (start 118.4 63.689998) (end 118.94 63.149998) (width 0.5) (layer F.Cu) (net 2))
 (segment (start 118.4 68.030002) (end 118.4 63.689998) (width 0.5) (layer F.Cu) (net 2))
 (segment (start 120.396 70.664) (end 117.2 73.86) (width 0.5) (layer F.Cu) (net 2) (status 30))
 (segment (start 120.396 69.944) (end 120.396 70.664) (width 0.5) (layer F.Cu) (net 2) (status 20))
 (segment (start 129.910012 72.810812) (end 130.048 72.9488) (width 0.5) (layer F.Cu) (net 2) (status 30))
 (segment (start 129.910012 68.08799) (end 129.910012 72.810812) (width 0.5) (layer F.Cu) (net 2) (status 20))
 (via (at 130.72 78.16) (size 0.8) (drill 0.4) (layers F.Cu B.Cu) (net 2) (status 30))
 (segment (start 130.72 93.0842) (end 131.2348 93.599) (width 0.5) (layer B.Cu) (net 2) (status 30))
 (segment (start 130.72 78.16) (end 130.72 93.0842) (width 0.5) (layer B.Cu) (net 2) (status 20))
 (segment (start 123.572 68.072) (end 124.3 68.8) (width 0.5) (layer F.Cu) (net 2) (status 30))
 (segment (start 123.205 68.072) (end 123.572 68.072) (width 0.5) (layer F.Cu) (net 2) (status 30))
 (segment (start 126.255001 64.150001) (end 123.982001 64.150001) (width 0.5) (layer B.Cu) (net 2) (status 20))
 (segment (start 126.6 63.805002) (end 126.255001 64.150001) (width 0.5) (layer B.Cu) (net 2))
 (segment (start 126.6 62.8) (end 126.6 63.805002) (width 0.5) (layer B.Cu) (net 2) (status 10))
 (segment (start 123.982001 64.150001) (end 123.84 64.008) (width 0.5) (layer B.Cu) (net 2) (status 30))
 (segment (start 117.2 74.069998) (end 119.086162 75.95616) (width 0.5) (layer B.Cu) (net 2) (status 10))
 (segment (start 117.2 73.86) (end 117.2 74.069998) (width 0.5) (layer B.Cu) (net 2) (status 30))
 (segment (start 119.086162 75.95616) (end 121.57964 75.95616) (width 0.5) (layer B.Cu) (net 2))
 (segment (start 121.57964 75.95616) (end 125.485801 72.049999) (width 0.5) (layer B.Cu) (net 2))
 (segment (start 125.485801 72.049999) (end 130.078839 72.049999) (width 0.5) (layer B.Cu) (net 2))
 (segment (start 130.72 72.69116) (end 130.72 78.16) (width 0.5) (layer B.Cu) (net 2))
 (segment (start 130.078839 72.049999) (end 130.72 72.69116) (width 0.5) (layer B.Cu) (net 2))
 (segment (start 130.80548 78.07452) (end 130.72 78.16) (width 0.5) (layer F.Cu) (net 2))
 (segment (start 134.57452 78.07452) (end 130.80548 78.07452) (width 0.5) (layer F.Cu) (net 2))
 (via (at 132.2 75.4) (size 0.8) (drill 0.4) (layers F.Cu B.Cu) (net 9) (status 30))
 (via (at 133.33 93.67) (size 0.8) (drill 0.4) (layers F.Cu B.Cu) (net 9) (status 30))
 (via (at 134.36 93.36) (size 0.5) (drill 0.3) (layers F.Cu B.Cu) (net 9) (status 30))
 (via (at 134.39 93.97) (size 0.5) (drill 0.3) (layers F.Cu B.Cu) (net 9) (status 30))
 (segment (start 131.749999 92.089999) (end 133.33 93.67) (width 0.5) (layer B.Cu) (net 9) (status 20))
 (segment (start 131.749999 75.850001) (end 131.749999 92.089999) (width 0.5) (layer B.Cu) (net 9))
 (segment (start 132.2 75.4) (end 131.749999 75.850001) (width 0.5) (layer B.Cu) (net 9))
 (segment (start 119.045988 75.421008) (end 119.045988 74.855323) (width 0.5) (layer F.Cu) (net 9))
 (segment (start 131.58 93.67) (end 119.720001 81.810001) (width 0.5) (layer F.Cu) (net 9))
 (segment (start 133.33 93.67) (end 131.58 93.67) (width 0.5) (layer F.Cu) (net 9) (status 10))
 (segment (start 117.2 66.24) (end 118.567239 67.607239) (width 0.5) (layer B.Cu) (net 9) (status 10))
 (via (at 119.045988 74.855323) (size 0.8) (drill 0.4) (layers F.Cu B.Cu) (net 9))
 (segment (start 118.567239 74.376574) (end 119.045988 74.855323) (width 0.5) (layer B.Cu) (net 9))
 (segment (start 118.567239 67.607239) (end 118.567239 74.376574) (width 0.5) (layer B.Cu) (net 9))
 (segment (start 119.720001 81.810001) (end 119.720001 76.095021) (width 0.5) (layer F.Cu) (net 9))
 (segment (start 119.720001 76.095021) (end 119.045988 75.421008) (width 0.5) (layer F.Cu) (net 9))
 (via (at 118.1 79.7) (size 0.8) (drill 0.4) (layers F.Cu B.Cu) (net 17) (status 30))
 (segment (start 115.999999 77.599999) (end 118.1 79.7) (width 0.5) (layer B.Cu) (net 17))
 (segment (start 117.2 71.32) (end 115.999999 72.520001) (width 0.5) (layer B.Cu) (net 17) (status 10))
 (segment (start 115.999999 72.520001) (end 115.999999 77.599999) (width 0.5) (layer B.Cu) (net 17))
 (segment (start 117.739998 81.66) (end 118.12 81.66) (width 0.5) (layer F.Cu) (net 16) (status 30))
 (segment (start 115.999999 79.920001) (end 117.739998 81.66) (width 0.5) (layer F.Cu) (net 16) (status 20))
 (segment (start 115.999999 69.980001) (end 115.999999 79.920001) (width 0.5) (layer F.Cu) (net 16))
 (segment (start 117.2 68.78) (end 115.999999 69.980001) (width 0.5) (layer F.Cu) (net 16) (status 10))
 (via (at 134.4 75.4) (size 0.8) (drill 0.4) (layers F.Cu B.Cu) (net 15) (status 30))
 (segment (start 135.150001 76.150001) (end 135.150001 87.949999) (width 0.5) (layer B.Cu) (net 15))
 (segment (start 134.4 75.4) (end 135.150001 76.150001) (width 0.5) (layer B.Cu) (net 15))
 (segment (start 135.150001 87.949999) (end 133.4 89.7) (width 0.5) (layer B.Cu) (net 15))
 (segment (start 133.4 89.7) (end 133.3 89.8) (width 0.5) (layer B.Cu) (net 15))
 (via (at 133.4 89.7) (size 0.8) (drill 0.4) (layers F.Cu B.Cu) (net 15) (status 30))
 (segment (start 127.7874 77.0926) (end 126.72 78.16) (width 0.5) (layer F.Cu) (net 14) (status 20))
 (segment (start 127.7874 75.3488) (end 127.7874 77.0926) (width 0.5) (layer F.Cu) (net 14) (status 10))
 (segment (start 125.5268 75.368) (end 124.72 76.1748) (width 0.5) (layer F.Cu) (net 13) (status 10))
 (segment (start 124.72 76.1748) (end 124.72 78.16) (width 0.5) (layer F.Cu) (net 13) (status 20))
 (segment (start 125.5268 75.368) (end 125.5268 75.0443) (width 0.25) (layer F.Cu) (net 13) (status 30))
 (segment (start 120.446201 74.443799) (end 120.396 74.494) (width 0.25) (layer F.Cu) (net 13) (status 30))
 (segment (start 124.926299 74.443799) (end 120.446201 74.443799) (width 0.25) (layer F.Cu) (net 13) (status 20))
 (segment (start 125.5268 75.0443) (end 124.926299 74.443799) (width 0.25) (layer F.Cu) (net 13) (status 10))
 (via (at 131.6 64.6) (size 0.8) (drill 0.4) (layers F.Cu B.Cu) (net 5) (status 30))
 (segment (start 123 62) (end 125.7 62) (width 0.5) (layer F.Cu) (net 5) (status 10))
 (segment (start 125.7 62) (end 129.5 62) (width 0.5) (layer F.Cu) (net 5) (status 20))
 (via (at 125.7 62) (size 0.8) (drill 0.4) (layers F.Cu B.Cu) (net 5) (status 30))
 (segment (start 132.55 66.5) (end 131.2 65.15) (width 0.5) (layer B.Cu) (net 5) (status 30))
 (segment (start 133.4 66.5) (end 132.55 66.5) (width 0.5) (layer B.Cu) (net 5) (status 30))
 (segment (start 129.5 63.45) (end 129.5 62) (width 0.5) (layer B.Cu) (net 5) (status 20))
 (segment (start 131.2 65.15) (end 129.5 63.45) (width 0.5) (layer B.Cu) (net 5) (status 10))
 (segment (start 119.300001 63.899999) (end 119.169999 63.899999) (width 0.5) (layer F.Cu) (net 5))
 (via (at 119.300001 63.899999) (size 0.8) (drill 0.4) (layers F.Cu B.Cu) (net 5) (status 30))
 (segment (start 123 63.415) (end 122.4075 64.0075) (width 0.5) (layer B.Cu) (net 5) (status 20))
 (segment (start 123 62) (end 123 63.415) (width 0.5) (layer B.Cu) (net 5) (status 10))
 (segment (start 122.4075 64.0075) (end 122.385 64.03) (width 0.5) (layer B.Cu) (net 5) (status 30))
 (segment (start 119.407502 64.0075) (end 119.300001 63.899999) (width 0.5) (layer F.Cu) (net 5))
 (segment (start 122.4075 64.0075) (end 122.365 64.0075) (width 0.5) (layer F.Cu) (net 5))
 (segment (start 122.365 64.0075) (end 119.407502 64.0075) (width 0.5) (layer F.Cu) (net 5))
 (via (at 122.365 64.0075) (size 0.5) (drill 0.3) (layers F.Cu B.Cu) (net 5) (status 30))
 (segment (start 130.048 76.832) (end 128.72 78.16) (width 0.5) (layer F.Cu) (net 12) (status 20))
 (segment (start 130.048 75.3488) (end 130.048 76.832) (width 0.5) (layer F.Cu) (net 12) (status 10))
 (via (at 120.2 67.2) (size 0.8) (drill 0.4) (layers F.Cu B.Cu) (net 6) (status 30))
 (segment (start 126.057603 73.993801) (end 122.393801 73.993801) (width 0.25) (layer F.Cu) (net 7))
 (segment (start 126.501801 74.437999) (end 126.057603 73.993801) (width 0.25) (layer F.Cu) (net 7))
 (segment (start 126.501801 76.298001) (end 126.501801 74.437999) (width 0.25) (layer F.Cu) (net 7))
 (segment (start 125.994999 78.690003) (end 125.994999 76.804803) (width 0.25) (layer F.Cu) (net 7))
 (segment (start 125.400001 79.285001) (end 125.994999 78.690003) (width 0.25) (layer F.Cu) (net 7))
 (segment (start 123.845001 79.285001) (end 125.400001 79.285001) (width 0.25) (layer F.Cu) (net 7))
 (segment (start 122.72 78.16) (end 123.845001 79.285001) (width 0.25) (layer F.Cu) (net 7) (status 10))
 (segment (start 125.994999 76.804803) (end 126.501801 76.298001) (width 0.25) (layer F.Cu) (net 7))
 (segment (start 122.393801 73.993801) (end 122.2 73.8) (width 0.25) (layer F.Cu) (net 7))
 (segment (start 122.2 73.8) (end 122.2 70.3) (width 0.25) (layer F.Cu) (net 7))
 (via (at 122.2 70.3) (size 0.8) (drill 0.4) (layers F.Cu B.Cu) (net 7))
 (segment (start 122.2 68.15) (end 122.021 67.971) (width 0.25) (layer B.Cu) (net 7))
 (segment (start 122.2 70.3) (end 122.2 68.15) (width 0.25) (layer B.Cu) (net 7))
 (segment (start 122.021 67.971) (end 121.15 67.1) (width 0.25) (layer B.Cu) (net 7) (status 20))
 (via (at 122.021 67.971) (size 0.5) (drill 0.3) (layers F.Cu B.Cu) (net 7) (status 30))
 (segment (start 126.492 69.9268) (end 123.4 73.0188) (width 0.5) (layer F.Cu) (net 1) (status 20))
 (segment (start 126.492 69.088) (end 126.492 69.9268) (width 0.5) (layer F.Cu) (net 1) (status 10))
 (segment (start 123.4 75.48) (end 120.72 78.16) (width 0.5) (layer F.Cu) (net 10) (status 30))
 (segment (start 123.4 75.4188) (end 123.4 75.48) (width 0.5) (layer F.Cu) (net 10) (status 30))
 (via (at 117.8 62.5) (size 0.8) (drill 0.4) (layers F.Cu B.Cu) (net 11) (status 30))
 (segment (start 123 66.5) (end 129.5 66.5) (width 0.5) (layer F.Cu) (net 8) (status 30))
 (segment (start 120.5 72.6) (end 121.7 72.6) (width 0.5) (layer B.Cu) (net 8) (status 10))
 (segment (start 123 71.3) (end 123 66.5) (width 0.5) (layer B.Cu) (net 8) (status 20))
 (segment (start 121.7 72.6) (end 123 71.3) (width 0.5) (layer B.Cu) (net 8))
 (segment (start 121.15 63.45) (end 121.15 64.5) (width 0.5) (layer B.Cu) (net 8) (status 20))
 (segment (start 120.3 62.6) (end 121.15 63.45) (width 0.5) (layer B.Cu) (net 8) (status 10))
 (segment (start 121.15 64.65) (end 123 66.5) (width 0.5) (layer B.Cu) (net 8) (status 30))
 (segment (start 121.15 64.5) (end 121.15 64.65) (width 0.5) (layer B.Cu) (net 8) (status 30))
 (segment (start 120.550001 65.149999) (end 126.050001 65.149999) (width 0.5) (layer F.Cu) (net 4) (status 10))
 (segment (start 120.3 65.4) (end 120.550001 65.149999) (width 0.5) (layer F.Cu) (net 4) (status 30))
 (segment (start 126.050001 65.149999) (end 127.55 63.65) (width 0.5) (layer F.Cu) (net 4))
 (segment (start 127.55 63.65) (end 127.6 63.6) (width 0.5) (layer F.Cu) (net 4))
 (via (at 127.55 63.65) (size 0.8) (drill 0.4) (layers F.Cu B.Cu) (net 4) (status 30)))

